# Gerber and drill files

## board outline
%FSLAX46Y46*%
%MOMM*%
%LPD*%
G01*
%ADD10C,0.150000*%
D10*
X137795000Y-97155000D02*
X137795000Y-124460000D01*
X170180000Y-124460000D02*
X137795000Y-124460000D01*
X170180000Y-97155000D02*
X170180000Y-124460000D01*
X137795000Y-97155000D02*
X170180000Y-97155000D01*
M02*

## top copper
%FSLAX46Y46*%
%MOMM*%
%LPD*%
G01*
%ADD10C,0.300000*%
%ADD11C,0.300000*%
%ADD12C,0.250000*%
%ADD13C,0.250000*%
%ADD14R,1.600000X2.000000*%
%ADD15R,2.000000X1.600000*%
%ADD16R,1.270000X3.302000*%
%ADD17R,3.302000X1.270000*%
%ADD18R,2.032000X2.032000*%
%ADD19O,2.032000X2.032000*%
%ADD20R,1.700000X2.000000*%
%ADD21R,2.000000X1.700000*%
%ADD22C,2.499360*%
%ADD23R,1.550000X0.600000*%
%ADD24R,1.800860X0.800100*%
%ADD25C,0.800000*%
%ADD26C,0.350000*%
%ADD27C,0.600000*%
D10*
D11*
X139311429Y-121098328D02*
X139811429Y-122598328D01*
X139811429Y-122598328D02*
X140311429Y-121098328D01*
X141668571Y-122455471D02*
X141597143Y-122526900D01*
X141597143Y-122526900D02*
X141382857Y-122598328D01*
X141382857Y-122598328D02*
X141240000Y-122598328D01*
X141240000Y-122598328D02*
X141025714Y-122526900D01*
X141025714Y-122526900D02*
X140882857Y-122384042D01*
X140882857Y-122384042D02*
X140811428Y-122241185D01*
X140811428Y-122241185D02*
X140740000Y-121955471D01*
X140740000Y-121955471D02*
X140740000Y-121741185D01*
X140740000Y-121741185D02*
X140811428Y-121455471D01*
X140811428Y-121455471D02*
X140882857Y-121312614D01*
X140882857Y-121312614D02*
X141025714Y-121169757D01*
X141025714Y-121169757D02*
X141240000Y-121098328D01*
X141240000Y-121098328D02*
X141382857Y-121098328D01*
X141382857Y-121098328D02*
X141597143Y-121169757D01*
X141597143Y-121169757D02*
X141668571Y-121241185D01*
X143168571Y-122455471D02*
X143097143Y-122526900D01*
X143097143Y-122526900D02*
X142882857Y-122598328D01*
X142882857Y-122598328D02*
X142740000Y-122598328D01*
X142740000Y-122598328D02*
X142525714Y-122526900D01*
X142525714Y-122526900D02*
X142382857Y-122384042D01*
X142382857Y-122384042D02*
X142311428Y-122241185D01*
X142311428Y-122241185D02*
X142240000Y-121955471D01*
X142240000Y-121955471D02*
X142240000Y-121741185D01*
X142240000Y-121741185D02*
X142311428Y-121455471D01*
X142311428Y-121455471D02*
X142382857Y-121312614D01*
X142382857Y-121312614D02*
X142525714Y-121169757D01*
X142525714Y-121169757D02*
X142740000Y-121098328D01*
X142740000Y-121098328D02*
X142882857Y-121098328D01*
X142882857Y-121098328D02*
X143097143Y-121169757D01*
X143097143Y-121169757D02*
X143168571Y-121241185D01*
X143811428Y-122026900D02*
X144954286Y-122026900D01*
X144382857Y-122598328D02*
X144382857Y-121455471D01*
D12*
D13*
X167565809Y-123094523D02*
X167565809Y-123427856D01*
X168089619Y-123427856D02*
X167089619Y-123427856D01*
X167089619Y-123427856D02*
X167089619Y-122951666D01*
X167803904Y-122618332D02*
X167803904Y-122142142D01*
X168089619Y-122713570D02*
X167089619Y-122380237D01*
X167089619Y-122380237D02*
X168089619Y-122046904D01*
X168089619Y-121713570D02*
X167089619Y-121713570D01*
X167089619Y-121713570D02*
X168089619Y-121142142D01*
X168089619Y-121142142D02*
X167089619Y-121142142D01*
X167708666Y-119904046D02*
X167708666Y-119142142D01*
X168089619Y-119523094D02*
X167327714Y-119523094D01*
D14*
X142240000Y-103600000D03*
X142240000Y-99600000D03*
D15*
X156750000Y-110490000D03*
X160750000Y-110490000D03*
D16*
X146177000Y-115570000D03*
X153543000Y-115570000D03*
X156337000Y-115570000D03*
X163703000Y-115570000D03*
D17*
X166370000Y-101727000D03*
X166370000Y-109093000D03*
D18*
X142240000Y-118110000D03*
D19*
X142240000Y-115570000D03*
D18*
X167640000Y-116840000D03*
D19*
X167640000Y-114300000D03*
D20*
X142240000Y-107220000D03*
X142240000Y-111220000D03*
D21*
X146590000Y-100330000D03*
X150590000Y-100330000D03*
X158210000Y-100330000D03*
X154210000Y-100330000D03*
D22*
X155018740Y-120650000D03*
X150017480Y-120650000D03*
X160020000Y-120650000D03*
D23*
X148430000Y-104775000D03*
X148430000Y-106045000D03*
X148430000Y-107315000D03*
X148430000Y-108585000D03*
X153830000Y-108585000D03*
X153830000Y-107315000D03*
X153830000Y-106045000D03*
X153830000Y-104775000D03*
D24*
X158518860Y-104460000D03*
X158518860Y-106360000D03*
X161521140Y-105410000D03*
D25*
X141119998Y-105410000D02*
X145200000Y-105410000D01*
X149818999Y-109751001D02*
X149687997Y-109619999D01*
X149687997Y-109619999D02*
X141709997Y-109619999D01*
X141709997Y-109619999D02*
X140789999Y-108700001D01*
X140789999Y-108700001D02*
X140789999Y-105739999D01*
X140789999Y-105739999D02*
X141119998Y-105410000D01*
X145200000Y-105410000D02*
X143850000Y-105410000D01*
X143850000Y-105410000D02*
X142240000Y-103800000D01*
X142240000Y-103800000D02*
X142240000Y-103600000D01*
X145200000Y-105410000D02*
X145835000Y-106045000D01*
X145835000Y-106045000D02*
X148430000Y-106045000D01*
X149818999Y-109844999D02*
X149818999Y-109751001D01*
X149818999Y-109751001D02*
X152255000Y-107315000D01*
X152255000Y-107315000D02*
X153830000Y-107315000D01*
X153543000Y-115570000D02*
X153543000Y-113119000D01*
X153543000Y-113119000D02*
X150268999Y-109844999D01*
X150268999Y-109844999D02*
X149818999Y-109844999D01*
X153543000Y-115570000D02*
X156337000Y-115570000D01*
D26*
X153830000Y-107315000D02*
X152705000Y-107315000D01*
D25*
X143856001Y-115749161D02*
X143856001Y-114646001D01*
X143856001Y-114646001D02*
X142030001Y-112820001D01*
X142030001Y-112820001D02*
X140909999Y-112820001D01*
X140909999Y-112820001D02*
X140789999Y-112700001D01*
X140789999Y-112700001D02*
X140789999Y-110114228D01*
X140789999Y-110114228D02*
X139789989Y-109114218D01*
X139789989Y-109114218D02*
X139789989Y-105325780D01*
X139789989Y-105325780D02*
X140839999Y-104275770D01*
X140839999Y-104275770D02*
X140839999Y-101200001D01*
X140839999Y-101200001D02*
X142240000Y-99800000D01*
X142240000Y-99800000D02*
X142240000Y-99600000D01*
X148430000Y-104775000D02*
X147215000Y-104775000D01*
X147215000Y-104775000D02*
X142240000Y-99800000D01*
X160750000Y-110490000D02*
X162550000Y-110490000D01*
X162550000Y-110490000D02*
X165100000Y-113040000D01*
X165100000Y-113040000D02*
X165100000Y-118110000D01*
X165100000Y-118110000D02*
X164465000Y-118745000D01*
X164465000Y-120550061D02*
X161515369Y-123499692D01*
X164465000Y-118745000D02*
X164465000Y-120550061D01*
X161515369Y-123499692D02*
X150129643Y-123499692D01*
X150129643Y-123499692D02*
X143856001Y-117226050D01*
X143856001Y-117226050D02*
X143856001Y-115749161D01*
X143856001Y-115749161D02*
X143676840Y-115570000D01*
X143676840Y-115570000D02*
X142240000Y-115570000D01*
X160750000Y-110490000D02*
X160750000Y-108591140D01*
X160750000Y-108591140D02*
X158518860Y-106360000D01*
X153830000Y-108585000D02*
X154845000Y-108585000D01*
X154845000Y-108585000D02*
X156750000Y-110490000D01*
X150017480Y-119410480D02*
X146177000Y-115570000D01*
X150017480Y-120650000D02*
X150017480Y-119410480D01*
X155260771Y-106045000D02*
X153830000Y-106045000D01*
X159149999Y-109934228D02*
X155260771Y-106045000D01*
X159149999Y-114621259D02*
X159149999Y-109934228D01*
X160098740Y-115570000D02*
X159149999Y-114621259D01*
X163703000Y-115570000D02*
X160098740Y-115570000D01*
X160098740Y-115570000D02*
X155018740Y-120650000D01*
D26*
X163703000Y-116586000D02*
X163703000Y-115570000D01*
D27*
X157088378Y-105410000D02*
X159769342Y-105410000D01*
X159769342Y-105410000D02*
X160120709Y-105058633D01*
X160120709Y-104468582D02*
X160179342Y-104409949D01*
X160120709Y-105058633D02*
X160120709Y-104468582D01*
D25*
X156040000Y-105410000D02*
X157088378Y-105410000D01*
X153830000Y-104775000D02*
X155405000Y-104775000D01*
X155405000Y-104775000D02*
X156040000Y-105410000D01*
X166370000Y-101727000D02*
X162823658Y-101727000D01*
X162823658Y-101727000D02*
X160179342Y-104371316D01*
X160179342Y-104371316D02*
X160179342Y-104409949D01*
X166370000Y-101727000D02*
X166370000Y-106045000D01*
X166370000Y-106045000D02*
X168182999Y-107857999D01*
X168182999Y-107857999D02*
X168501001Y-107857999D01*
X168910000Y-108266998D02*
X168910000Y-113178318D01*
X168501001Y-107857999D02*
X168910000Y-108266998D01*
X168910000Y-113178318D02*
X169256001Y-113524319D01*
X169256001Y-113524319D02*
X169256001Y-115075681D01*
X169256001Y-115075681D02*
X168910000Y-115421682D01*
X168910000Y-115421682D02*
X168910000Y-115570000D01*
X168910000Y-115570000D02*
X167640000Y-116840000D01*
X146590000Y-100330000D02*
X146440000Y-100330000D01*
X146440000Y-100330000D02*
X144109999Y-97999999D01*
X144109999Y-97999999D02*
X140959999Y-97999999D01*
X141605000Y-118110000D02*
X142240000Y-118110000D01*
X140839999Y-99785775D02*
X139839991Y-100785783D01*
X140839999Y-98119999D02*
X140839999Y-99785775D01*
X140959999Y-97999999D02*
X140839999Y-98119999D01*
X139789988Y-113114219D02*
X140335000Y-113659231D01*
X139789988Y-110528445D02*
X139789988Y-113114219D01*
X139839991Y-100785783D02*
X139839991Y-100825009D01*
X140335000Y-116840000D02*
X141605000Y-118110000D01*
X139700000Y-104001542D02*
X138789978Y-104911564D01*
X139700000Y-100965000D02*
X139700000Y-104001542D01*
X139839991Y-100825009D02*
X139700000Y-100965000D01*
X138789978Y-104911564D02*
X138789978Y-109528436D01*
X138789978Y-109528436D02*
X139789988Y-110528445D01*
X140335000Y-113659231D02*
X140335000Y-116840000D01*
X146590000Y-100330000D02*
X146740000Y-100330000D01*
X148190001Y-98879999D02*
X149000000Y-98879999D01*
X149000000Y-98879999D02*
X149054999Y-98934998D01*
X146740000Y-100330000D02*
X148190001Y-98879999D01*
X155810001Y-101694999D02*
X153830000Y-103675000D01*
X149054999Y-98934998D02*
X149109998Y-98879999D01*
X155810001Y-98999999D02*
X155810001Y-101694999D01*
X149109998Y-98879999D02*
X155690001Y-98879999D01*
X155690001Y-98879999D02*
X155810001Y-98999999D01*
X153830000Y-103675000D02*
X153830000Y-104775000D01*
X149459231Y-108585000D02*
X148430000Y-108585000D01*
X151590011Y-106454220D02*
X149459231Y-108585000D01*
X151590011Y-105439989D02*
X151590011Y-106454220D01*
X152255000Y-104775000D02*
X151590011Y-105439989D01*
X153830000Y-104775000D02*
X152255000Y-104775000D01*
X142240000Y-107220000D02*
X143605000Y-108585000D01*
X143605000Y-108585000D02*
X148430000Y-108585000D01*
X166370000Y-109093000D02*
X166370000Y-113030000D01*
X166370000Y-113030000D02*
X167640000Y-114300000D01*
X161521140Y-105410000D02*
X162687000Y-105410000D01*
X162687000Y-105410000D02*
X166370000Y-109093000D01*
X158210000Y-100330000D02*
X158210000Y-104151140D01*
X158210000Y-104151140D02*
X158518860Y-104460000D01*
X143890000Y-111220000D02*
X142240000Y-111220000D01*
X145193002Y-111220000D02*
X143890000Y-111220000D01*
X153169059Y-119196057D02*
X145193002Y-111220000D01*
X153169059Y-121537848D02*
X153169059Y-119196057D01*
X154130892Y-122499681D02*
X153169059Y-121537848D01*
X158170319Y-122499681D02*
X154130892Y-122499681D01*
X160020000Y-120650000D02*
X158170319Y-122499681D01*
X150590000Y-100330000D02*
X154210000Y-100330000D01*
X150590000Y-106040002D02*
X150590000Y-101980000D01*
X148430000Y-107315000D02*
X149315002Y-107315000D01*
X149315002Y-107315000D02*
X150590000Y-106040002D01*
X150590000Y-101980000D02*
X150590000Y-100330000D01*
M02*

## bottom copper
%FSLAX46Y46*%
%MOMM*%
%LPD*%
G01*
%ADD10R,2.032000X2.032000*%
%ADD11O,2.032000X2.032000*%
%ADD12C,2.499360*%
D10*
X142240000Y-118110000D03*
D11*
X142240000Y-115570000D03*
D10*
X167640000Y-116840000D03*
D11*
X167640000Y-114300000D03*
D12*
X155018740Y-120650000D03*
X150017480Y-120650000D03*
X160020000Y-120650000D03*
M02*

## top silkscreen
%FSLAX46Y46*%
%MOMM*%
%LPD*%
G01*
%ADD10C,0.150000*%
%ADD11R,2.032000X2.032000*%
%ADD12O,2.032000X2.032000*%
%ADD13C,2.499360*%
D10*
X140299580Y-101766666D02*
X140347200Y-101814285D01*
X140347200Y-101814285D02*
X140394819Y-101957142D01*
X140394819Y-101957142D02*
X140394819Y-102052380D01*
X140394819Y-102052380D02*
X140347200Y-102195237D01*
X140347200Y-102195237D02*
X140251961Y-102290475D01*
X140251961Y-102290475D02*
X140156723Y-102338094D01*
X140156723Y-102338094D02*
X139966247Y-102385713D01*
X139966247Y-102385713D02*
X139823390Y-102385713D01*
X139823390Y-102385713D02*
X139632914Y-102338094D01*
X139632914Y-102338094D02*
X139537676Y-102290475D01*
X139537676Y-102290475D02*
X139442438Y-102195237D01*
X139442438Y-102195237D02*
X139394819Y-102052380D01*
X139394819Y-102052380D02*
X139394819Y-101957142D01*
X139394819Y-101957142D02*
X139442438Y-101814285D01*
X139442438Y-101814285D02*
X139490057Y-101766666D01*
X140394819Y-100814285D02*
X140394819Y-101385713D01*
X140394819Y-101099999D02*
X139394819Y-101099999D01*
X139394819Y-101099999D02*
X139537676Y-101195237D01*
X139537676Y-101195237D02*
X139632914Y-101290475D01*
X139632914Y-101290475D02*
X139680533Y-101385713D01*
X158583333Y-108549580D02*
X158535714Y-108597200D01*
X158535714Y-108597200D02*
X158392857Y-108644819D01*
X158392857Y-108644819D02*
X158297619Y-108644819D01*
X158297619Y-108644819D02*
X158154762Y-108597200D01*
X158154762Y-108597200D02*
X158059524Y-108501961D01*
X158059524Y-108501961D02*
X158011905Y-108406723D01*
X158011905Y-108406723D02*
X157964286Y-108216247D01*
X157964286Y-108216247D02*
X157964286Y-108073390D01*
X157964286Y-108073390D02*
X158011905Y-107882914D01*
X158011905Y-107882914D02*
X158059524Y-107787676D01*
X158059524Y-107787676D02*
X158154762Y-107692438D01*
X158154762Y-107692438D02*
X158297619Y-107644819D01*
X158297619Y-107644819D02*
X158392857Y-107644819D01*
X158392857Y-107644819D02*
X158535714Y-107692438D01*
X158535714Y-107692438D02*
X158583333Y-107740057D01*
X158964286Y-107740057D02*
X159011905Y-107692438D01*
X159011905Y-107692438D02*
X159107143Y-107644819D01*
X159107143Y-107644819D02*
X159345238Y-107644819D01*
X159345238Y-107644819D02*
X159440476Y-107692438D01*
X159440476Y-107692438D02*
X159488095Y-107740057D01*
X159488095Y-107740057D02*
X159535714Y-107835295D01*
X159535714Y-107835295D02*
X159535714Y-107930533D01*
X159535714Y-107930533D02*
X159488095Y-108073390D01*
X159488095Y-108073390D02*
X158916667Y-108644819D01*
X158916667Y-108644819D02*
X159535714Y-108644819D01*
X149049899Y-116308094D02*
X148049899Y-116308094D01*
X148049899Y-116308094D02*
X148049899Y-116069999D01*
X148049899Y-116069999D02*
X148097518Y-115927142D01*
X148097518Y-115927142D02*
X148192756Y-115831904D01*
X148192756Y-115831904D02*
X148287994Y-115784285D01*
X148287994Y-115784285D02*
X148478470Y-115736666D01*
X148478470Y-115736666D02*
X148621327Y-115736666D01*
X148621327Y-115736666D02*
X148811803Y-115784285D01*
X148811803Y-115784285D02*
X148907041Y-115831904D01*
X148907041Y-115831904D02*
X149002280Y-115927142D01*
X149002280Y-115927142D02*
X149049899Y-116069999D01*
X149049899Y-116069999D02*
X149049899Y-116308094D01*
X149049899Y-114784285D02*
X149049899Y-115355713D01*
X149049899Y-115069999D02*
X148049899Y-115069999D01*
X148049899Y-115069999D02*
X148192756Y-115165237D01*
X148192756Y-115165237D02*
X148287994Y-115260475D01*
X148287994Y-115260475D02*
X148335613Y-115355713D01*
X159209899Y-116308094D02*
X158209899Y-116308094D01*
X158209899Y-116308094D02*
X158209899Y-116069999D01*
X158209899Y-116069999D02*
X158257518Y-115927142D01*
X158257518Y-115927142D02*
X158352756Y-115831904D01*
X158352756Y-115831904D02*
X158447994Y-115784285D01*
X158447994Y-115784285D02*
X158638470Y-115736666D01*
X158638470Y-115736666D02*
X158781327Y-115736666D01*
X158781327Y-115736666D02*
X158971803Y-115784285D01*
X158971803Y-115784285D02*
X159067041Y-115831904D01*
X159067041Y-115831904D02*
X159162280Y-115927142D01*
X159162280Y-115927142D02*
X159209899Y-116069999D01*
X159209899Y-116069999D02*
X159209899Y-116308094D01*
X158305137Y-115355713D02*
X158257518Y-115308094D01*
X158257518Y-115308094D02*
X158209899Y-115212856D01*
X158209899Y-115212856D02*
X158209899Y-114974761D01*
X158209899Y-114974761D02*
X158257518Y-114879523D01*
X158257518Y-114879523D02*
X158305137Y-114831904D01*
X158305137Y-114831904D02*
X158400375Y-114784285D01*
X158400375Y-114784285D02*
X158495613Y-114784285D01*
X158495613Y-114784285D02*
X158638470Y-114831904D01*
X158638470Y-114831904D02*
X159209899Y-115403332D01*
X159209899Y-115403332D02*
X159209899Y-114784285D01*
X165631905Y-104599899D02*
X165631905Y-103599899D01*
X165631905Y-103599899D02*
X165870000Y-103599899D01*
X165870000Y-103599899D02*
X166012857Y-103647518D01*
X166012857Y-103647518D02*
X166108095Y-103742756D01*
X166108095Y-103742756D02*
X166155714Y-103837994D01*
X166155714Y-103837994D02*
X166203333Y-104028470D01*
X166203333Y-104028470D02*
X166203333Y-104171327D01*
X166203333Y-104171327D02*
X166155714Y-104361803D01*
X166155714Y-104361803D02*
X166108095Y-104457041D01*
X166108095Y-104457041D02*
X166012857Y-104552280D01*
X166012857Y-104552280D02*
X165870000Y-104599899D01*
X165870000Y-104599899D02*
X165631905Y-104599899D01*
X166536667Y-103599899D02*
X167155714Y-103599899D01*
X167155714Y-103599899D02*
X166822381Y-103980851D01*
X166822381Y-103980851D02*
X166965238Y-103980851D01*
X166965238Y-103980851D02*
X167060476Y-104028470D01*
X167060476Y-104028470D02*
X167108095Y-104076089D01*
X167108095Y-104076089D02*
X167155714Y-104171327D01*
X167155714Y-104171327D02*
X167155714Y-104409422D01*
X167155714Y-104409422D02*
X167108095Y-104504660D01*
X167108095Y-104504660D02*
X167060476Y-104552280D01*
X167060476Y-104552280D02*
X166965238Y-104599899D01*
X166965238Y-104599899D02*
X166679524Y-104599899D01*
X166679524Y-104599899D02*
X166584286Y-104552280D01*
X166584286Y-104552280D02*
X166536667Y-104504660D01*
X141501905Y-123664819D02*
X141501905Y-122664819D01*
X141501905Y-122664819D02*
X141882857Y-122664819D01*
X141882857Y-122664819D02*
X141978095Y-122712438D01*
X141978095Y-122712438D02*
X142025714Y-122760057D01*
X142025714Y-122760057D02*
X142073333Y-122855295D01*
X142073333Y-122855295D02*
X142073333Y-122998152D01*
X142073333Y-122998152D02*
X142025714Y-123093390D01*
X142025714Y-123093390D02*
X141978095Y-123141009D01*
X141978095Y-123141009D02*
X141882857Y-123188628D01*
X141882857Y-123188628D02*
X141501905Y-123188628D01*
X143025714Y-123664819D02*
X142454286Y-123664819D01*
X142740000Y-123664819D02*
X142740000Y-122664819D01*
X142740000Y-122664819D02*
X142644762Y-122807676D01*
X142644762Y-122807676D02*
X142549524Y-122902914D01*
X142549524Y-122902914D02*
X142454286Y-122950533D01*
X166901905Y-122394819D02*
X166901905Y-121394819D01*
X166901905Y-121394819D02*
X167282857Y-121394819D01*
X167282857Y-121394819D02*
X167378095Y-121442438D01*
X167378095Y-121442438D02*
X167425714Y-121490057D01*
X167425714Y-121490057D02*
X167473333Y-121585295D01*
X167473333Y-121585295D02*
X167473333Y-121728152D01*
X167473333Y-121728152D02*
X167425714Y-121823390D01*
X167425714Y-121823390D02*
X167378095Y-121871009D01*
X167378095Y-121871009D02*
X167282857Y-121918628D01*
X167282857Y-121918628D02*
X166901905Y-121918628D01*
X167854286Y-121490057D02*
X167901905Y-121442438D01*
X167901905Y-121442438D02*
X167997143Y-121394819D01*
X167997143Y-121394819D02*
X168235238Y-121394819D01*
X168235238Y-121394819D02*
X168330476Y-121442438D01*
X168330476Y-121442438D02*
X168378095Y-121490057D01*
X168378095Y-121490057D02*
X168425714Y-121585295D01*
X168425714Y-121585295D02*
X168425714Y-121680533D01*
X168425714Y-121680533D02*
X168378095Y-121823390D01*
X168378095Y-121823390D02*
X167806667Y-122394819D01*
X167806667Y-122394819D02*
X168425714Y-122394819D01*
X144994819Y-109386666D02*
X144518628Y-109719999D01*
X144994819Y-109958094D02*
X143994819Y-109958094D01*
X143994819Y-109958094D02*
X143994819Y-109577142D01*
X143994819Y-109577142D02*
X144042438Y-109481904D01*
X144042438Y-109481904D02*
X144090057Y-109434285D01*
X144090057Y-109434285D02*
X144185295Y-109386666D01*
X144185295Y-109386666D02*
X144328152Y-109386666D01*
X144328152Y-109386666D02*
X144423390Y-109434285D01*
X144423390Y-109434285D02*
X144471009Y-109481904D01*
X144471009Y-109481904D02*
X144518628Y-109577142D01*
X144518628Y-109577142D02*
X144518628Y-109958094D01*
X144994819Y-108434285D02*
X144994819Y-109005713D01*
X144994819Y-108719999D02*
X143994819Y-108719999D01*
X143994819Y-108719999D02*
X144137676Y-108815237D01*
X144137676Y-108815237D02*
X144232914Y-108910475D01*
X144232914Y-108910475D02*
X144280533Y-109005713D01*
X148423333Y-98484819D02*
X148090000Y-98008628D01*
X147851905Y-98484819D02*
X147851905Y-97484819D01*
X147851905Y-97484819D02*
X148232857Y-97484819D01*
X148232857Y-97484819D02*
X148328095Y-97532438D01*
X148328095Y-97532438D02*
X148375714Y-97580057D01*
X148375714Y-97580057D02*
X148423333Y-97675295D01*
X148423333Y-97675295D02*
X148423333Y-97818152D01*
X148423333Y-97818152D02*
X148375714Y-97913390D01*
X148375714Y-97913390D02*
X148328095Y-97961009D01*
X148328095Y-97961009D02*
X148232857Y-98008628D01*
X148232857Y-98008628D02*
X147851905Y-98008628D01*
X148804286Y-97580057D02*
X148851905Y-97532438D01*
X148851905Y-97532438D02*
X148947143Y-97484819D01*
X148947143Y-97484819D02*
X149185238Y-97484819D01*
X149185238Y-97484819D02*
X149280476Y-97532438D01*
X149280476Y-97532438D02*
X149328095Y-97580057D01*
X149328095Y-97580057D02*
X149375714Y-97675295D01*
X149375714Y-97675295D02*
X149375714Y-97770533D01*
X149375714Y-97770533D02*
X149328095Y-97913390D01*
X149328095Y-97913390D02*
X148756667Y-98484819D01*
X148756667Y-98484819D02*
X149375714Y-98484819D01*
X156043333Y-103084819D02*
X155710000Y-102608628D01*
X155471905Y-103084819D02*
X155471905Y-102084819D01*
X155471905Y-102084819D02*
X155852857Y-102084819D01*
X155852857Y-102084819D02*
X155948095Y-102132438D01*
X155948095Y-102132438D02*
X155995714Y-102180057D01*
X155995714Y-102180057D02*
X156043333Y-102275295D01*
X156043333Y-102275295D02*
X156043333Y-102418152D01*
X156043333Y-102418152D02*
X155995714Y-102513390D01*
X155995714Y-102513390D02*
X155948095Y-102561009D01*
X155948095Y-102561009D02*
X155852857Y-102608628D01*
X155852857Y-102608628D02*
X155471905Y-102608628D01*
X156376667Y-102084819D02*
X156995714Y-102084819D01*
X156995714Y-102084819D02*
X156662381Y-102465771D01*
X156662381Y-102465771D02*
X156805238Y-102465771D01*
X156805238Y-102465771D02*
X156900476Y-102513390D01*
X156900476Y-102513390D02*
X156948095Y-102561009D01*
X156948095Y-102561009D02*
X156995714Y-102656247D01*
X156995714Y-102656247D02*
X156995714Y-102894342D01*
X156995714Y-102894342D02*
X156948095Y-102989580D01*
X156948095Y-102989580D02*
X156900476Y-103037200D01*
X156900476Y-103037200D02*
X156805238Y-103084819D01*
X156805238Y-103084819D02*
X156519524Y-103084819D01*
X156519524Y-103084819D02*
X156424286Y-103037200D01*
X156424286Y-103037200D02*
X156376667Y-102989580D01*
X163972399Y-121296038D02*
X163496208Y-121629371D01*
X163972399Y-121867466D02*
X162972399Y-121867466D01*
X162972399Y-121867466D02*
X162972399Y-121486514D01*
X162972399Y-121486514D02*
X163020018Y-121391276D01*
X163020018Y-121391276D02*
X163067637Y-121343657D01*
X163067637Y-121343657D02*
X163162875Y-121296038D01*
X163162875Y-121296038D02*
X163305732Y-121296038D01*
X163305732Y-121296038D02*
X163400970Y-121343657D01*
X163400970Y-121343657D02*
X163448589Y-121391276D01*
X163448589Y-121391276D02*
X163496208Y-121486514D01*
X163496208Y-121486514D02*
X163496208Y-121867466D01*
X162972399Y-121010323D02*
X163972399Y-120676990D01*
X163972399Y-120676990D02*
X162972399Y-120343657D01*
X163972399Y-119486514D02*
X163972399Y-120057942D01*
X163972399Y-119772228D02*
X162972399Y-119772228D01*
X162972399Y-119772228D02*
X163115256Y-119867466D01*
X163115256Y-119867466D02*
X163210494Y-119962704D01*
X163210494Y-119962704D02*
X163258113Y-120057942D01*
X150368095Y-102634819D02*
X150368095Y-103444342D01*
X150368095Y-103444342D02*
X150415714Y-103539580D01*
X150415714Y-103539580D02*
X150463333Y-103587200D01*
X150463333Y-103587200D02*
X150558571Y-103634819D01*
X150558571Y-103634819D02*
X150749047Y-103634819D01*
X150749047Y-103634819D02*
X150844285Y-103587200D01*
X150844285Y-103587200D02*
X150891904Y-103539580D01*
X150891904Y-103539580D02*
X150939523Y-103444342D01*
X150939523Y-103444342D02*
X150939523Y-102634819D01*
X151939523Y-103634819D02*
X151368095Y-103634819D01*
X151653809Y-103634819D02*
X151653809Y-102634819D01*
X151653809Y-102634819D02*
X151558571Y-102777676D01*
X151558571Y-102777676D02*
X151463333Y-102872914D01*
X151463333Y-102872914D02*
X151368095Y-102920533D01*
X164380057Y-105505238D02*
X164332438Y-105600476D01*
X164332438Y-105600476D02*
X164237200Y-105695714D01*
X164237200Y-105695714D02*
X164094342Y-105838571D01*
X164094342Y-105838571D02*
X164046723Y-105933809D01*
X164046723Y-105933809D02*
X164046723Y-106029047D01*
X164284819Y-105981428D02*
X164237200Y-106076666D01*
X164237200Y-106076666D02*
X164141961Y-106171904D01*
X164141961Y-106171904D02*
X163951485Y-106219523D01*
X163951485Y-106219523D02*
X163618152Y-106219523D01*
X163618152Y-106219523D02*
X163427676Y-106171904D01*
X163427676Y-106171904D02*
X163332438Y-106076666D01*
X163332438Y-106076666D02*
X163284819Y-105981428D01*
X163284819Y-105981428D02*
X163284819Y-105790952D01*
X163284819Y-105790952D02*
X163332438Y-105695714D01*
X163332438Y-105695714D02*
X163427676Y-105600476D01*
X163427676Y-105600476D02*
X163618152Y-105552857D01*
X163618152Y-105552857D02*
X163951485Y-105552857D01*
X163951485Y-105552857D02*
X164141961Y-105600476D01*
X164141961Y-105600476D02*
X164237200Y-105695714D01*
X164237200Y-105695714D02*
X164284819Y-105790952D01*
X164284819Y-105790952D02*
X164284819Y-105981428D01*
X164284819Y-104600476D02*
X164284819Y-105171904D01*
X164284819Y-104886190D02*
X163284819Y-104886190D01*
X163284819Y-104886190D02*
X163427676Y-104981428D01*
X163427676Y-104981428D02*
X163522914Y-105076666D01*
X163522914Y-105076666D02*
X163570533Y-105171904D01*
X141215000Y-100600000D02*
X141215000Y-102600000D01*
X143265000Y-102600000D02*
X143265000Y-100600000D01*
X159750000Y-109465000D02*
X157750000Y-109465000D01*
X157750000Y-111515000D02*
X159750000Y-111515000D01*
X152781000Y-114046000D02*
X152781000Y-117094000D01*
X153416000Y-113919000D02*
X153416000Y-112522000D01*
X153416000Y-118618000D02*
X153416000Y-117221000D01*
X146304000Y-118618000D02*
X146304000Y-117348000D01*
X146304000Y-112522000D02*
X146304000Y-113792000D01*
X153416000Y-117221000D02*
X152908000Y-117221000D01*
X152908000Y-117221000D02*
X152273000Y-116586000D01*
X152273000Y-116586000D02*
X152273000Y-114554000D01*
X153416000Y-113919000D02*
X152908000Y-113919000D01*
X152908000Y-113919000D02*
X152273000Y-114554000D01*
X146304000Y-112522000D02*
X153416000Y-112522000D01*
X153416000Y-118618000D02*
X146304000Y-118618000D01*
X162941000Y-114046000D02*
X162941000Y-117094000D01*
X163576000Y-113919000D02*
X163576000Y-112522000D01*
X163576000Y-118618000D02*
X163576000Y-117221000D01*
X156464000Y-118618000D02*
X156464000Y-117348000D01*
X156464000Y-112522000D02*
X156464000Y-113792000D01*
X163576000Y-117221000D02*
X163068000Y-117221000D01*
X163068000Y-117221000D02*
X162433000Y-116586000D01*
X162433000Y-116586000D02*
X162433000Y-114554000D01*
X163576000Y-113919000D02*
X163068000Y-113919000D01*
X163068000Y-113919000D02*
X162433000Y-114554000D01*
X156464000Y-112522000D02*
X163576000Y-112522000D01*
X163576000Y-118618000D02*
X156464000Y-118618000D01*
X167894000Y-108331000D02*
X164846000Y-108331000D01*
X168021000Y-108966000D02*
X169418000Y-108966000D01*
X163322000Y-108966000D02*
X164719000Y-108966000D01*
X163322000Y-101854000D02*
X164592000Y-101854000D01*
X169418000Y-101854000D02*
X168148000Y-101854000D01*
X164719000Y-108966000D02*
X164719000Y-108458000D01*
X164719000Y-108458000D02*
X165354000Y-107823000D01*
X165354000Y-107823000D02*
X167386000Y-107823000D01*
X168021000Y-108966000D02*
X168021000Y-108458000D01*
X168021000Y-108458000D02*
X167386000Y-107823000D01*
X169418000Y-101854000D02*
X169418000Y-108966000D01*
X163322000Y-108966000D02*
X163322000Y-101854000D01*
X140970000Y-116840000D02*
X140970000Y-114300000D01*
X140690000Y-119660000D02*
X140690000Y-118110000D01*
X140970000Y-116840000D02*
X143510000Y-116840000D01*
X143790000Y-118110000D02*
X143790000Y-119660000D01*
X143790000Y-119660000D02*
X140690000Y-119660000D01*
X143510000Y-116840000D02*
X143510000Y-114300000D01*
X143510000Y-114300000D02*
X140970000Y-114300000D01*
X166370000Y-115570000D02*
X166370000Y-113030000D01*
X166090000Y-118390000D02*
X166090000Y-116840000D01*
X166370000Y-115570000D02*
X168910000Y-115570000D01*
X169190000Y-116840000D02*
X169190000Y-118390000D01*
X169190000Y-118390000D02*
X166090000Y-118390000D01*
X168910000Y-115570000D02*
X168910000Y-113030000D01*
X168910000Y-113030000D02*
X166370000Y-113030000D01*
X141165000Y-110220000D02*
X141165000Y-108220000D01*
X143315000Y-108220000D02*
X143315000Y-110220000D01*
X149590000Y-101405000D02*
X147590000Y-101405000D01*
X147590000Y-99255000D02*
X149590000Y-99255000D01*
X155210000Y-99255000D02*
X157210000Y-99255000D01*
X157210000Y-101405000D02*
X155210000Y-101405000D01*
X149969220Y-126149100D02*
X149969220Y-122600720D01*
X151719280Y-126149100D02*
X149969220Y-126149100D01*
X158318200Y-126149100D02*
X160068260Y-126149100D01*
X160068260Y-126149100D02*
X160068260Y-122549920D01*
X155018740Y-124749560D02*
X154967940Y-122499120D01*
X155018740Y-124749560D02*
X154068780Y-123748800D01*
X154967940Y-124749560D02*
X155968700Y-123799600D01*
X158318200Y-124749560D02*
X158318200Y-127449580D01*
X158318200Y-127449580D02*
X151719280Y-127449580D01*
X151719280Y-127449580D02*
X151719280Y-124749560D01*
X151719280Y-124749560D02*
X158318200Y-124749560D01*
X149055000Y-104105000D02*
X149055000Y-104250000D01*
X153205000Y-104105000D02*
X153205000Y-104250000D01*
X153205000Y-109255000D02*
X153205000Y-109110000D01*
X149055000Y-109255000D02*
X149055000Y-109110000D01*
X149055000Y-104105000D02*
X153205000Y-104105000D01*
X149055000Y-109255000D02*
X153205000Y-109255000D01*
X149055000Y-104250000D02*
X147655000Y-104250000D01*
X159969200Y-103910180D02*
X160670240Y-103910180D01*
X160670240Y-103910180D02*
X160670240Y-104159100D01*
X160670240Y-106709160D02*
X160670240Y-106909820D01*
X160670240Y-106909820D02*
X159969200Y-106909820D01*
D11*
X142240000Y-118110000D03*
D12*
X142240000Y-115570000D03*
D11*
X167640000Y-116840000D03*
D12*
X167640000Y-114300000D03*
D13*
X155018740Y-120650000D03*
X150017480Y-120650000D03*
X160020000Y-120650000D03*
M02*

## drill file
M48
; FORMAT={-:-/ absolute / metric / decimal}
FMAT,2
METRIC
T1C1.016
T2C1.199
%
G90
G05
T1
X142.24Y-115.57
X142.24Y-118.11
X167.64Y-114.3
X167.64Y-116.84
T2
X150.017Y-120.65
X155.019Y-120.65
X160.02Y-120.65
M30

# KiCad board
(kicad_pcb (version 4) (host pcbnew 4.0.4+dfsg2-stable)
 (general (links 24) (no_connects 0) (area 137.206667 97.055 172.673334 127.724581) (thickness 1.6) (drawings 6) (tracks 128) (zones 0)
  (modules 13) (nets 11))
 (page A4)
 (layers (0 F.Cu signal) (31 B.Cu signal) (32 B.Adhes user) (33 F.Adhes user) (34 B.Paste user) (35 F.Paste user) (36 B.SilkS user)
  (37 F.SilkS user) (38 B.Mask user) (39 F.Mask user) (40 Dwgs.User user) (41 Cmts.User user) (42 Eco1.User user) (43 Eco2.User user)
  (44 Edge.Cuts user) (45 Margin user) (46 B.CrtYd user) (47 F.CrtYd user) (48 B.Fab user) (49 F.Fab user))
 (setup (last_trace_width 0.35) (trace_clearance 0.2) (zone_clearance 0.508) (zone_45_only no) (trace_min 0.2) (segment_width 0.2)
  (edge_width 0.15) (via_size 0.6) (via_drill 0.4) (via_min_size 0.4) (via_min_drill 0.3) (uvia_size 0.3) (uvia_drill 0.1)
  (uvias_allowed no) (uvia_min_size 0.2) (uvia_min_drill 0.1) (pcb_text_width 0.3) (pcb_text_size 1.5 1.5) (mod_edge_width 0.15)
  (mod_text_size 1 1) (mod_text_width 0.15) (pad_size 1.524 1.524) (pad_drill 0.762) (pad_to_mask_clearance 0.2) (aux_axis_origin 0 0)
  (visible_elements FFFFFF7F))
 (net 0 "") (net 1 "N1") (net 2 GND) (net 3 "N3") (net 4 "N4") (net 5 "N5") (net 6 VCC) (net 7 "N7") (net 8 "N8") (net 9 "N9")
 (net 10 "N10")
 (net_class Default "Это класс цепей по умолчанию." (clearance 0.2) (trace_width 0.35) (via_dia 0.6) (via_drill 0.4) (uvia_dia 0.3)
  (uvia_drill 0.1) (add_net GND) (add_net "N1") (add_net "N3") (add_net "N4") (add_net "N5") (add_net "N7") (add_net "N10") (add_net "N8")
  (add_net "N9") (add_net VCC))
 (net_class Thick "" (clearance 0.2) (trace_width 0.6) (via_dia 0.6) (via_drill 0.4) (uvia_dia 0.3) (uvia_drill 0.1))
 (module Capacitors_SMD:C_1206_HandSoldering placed (layer F.Cu) (at 142.24 101.6 90)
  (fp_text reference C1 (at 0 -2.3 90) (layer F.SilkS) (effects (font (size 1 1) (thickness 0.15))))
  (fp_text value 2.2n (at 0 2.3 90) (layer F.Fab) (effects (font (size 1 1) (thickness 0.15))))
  (fp_line (start 1 -1.025) (end -1 -1.025) (layer F.SilkS) (width 0.15))
  (fp_line (start -1 1.025) (end 1 1.025) (layer F.SilkS) (width 0.15))
  (pad 1 smd rect (at -2 0 90) (size 2 1.6) (layers F.Cu F.Paste F.Mask) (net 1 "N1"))
  (pad 2 smd rect (at 2 0 90) (size 2 1.6) (layers F.Cu F.Paste F.Mask) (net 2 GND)))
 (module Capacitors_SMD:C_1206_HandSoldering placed (layer F.Cu) (at 158.75 110.49)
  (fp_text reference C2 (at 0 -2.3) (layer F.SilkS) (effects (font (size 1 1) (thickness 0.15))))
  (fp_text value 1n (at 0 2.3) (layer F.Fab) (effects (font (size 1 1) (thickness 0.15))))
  (fp_line (start 1 -1.025) (end -1 -1.025) (layer F.SilkS) (width 0.15))
  (fp_line (start -1 1.025) (end 1 1.025) (layer F.SilkS) (width 0.15))
  (pad 1 smd rect (at -2 0) (size 2 1.6) (layers F.Cu F.Paste F.Mask) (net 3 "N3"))
  (pad 2 smd rect (at 2 0) (size 2 1.6) (layers F.Cu F.Paste F.Mask) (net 2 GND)))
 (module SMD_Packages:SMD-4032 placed (layer F.Cu) (at 149.86 115.57)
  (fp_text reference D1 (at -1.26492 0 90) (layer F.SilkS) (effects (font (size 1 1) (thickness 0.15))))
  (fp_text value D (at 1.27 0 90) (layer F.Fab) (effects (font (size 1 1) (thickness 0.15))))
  (fp_line (start 2.921 -1.524) (end 2.921 1.524) (layer F.SilkS) (width 0.15))
  (fp_line (start 3.556 -1.651) (end 3.556 -3.048) (layer F.SilkS) (width 0.15))
  (fp_line (start 3.556 3.048) (end 3.556 1.651) (layer F.SilkS) (width 0.15))
  (fp_line (start -3.556 3.048) (end -3.556 1.778) (layer F.SilkS) (width 0.15))
  (fp_line (start -3.556 -3.048) (end -3.556 -1.778) (layer F.SilkS) (width 0.15))
  (fp_line (start 3.556 1.651) (end 3.048 1.651) (layer F.SilkS) (width 0.15))
  (fp_line (start 3.048 1.651) (end 2.413 1.016) (layer F.SilkS) (width 0.15))
  (fp_line (start 2.413 1.016) (end 2.413 -1.016) (layer F.SilkS) (width 0.15))
  (fp_line (start 3.556 -1.651) (end 3.048 -1.651) (layer F.SilkS) (width 0.15))
  (fp_line (start 3.048 -1.651) (end 2.413 -1.016) (layer F.SilkS) (width 0.15))
  (fp_line (start -3.556 -3.048) (end 3.556 -3.048) (layer F.SilkS) (width 0.15))
  (fp_line (start 3.556 3.048) (end -3.556 3.048) (layer F.SilkS) (width 0.15))
  (pad 1 smd rect (at -3.683 0) (size 1.27 3.302) (layers F.Cu F.Paste F.Mask) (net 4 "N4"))
  (pad 2 smd rect (at 3.683 0) (size 1.27 3.302) (layers F.Cu F.Paste F.Mask) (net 1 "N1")))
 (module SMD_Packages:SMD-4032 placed (layer F.Cu) (at 160.02 115.57)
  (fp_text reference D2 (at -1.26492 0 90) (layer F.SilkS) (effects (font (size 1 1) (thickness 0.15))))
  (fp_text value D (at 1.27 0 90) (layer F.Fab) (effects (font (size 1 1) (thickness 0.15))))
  (fp_line (start 2.921 -1.524) (end 2.921 1.524) (layer F.SilkS) (width 0.15))
  (fp_line (start 3.556 -1.651) (end 3.556 -3.048) (layer F.SilkS) (width 0.15))
  (fp_line (start 3.556 3.048) (end 3.556 1.651) (layer F.SilkS) (width 0.15))
  (fp_line (start -3.556 3.048) (end -3.556 1.778) (layer F.SilkS) (width 0.15))
  (fp_line (start -3.556 -3.048) (end -3.556 -1.778) (layer F.SilkS) (width 0.15))
  (fp_line (start 3.556 1.651) (end 3.048 1.651) (layer F.SilkS) (width 0.15))
  (fp_line (start 3.048 1.651) (end 2.413 1.016) (layer F.SilkS) (width 0.15))
  (fp_line (start 2.413 1.016) (end 2.413 -1.016) (layer F.SilkS) (width 0.15))
  (fp_line (start 3.556 -1.651) (end 3.048 -1.651) (layer F.SilkS) (width 0.15))
  (fp_line (start 3.048 -1.651) (end 2.413 -1.016) (layer F.SilkS) (width 0.15))
  (fp_line (start -3.556 -3.048) (end 3.556 -3.048) (layer F.SilkS) (width 0.15))
  (fp_line (start 3.556 3.048) (end -3.556 3.048) (layer F.SilkS) (width 0.15))
  (pad 1 smd rect (at -3.683 0) (size 1.27 3.302) (layers F.Cu F.Paste F.Mask) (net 1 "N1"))
  (pad 2 smd rect (at 3.683 0) (size 1.27 3.302) (layers F.Cu F.Paste F.Mask) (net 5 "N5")))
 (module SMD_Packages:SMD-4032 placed (layer F.Cu) (at 166.37 105.41 270)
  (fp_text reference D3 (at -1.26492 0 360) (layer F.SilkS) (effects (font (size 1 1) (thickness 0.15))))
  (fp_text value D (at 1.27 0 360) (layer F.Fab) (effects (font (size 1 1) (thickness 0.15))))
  (fp_line (start 2.921 -1.524) (end 2.921 1.524) (layer F.SilkS) (width 0.15))
  (fp_line (start 3.556 -1.651) (end 3.556 -3.048) (layer F.SilkS) (width 0.15))
  (fp_line (start 3.556 3.048) (end 3.556 1.651) (layer F.SilkS) (width 0.15))
  (fp_line (start -3.556 3.048) (end -3.556 1.778) (layer F.SilkS) (width 0.15))
  (fp_line (start -3.556 -3.048) (end -3.556 -1.778) (layer F.SilkS) (width 0.15))
  (fp_line (start 3.556 1.651) (end 3.048 1.651) (layer F.SilkS) (width 0.15))
  (fp_line (start 3.048 1.651) (end 2.413 1.016) (layer F.SilkS) (width 0.15))
  (fp_line (start 2.413 1.016) (end 2.413 -1.016) (layer F.SilkS) (width 0.15))
  (fp_line (start 3.556 -1.651) (end 3.048 -1.651) (layer F.SilkS) (width 0.15))
  (fp_line (start 3.048 -1.651) (end 2.413 -1.016) (layer F.SilkS) (width 0.15))
  (fp_line (start -3.556 -3.048) (end 3.556 -3.048) (layer F.SilkS) (width 0.15))
  (fp_line (start 3.556 3.048) (end -3.556 3.048) (layer F.SilkS) (width 0.15))
  (pad 1 smd rect (at -3.683 0 270) (size 1.27 3.302) (layers F.Cu F.Paste F.Mask) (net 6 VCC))
  (pad 2 smd rect (at 3.683 0 270) (size 1.27 3.302) (layers F.Cu F.Paste F.Mask) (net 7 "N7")))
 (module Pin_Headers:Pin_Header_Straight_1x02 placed (layer F.Cu) (at 142.24 118.11 180)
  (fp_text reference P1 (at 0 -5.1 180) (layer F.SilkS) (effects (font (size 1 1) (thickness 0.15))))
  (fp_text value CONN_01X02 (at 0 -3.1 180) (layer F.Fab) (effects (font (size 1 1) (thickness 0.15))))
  (fp_line (start 1.27 1.27) (end 1.27 3.81) (layer F.SilkS) (width 0.15))
  (fp_line (start 1.55 -1.55) (end 1.55 0) (layer F.SilkS) (width 0.15))
  (fp_line (start 1.27 1.27) (end -1.27 1.27) (layer F.SilkS) (width 0.15))
  (fp_line (start -1.55 0) (end -1.55 -1.55) (layer F.SilkS) (width 0.15))
  (fp_line (start -1.55 -1.55) (end 1.55 -1.55) (layer F.SilkS) (width 0.15))
  (fp_line (start -1.27 1.27) (end -1.27 3.81) (layer F.SilkS) (width 0.15))
  (fp_line (start -1.27 3.81) (end 1.27 3.81) (layer F.SilkS) (width 0.15))
  (pad 1 thru_hole rect (at 0 0 180) (size 2.032 2.032) (drill 1.016) (layers *.Cu *.Mask F.SilkS) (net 6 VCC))
  (pad 2 thru_hole oval (at 0 2.54 180) (size 2.032 2.032) (drill 1.016) (layers *.Cu *.Mask F.SilkS) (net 2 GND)))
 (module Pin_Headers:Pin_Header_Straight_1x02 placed (layer F.Cu) (at 167.64 116.84 180)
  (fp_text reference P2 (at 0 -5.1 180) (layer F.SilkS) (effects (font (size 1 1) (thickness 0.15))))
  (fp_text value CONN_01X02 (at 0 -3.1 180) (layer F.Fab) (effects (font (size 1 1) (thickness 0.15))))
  (fp_line (start 1.27 1.27) (end 1.27 3.81) (layer F.SilkS) (width 0.15))
  (fp_line (start 1.55 -1.55) (end 1.55 0) (layer F.SilkS) (width 0.15))
  (fp_line (start 1.27 1.27) (end -1.27 1.27) (layer F.SilkS) (width 0.15))
  (fp_line (start -1.55 0) (end -1.55 -1.55) (layer F.SilkS) (width 0.15))
  (fp_line (start -1.55 -1.55) (end 1.55 -1.55) (layer F.SilkS) (width 0.15))
  (fp_line (start -1.27 1.27) (end -1.27 3.81) (layer F.SilkS) (width 0.15))
  (fp_line (start -1.27 3.81) (end 1.27 3.81) (layer F.SilkS) (width 0.15))
  (pad 1 thru_hole rect (at 0 0 180) (size 2.032 2.032) (drill 1.016) (layers *.Cu *.Mask F.SilkS) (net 6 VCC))
  (pad 2 thru_hole oval (at 0 2.54 180) (size 2.032 2.032) (drill 1.016) (layers *.Cu *.Mask F.SilkS) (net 7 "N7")))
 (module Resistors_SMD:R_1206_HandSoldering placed (layer F.Cu) (at 142.24 109.22 270)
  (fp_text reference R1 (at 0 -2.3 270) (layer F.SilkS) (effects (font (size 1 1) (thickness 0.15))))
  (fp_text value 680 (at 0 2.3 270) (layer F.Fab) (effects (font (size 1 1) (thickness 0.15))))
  (fp_line (start 1 1.075) (end -1 1.075) (layer F.SilkS) (width 0.15))
  (fp_line (start -1 -1.075) (end 1 -1.075) (layer F.SilkS) (width 0.15))
  (pad 1 smd rect (at -2 0 270) (size 2 1.7) (layers F.Cu F.Paste F.Mask) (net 6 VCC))
  (pad 2 smd rect (at 2 0 270) (size 2 1.7) (layers F.Cu F.Paste F.Mask) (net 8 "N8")))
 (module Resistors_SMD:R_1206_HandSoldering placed (layer F.Cu) (at 148.59 100.33)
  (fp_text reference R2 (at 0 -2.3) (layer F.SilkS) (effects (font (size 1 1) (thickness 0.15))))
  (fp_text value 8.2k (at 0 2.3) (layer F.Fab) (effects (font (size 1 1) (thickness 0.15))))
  (fp_line (start 1 1.075) (end -1 1.075) (layer F.SilkS) (width 0.15))
  (fp_line (start -1 -1.075) (end 1 -1.075) (layer F.SilkS) (width 0.15))
  (pad 1 smd rect (at -2 0) (size 2 1.7) (layers F.Cu F.Paste F.Mask) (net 6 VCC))
  (pad 2 smd rect (at 2 0) (size 2 1.7) (layers F.Cu F.Paste F.Mask) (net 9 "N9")))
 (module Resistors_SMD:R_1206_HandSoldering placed (layer F.Cu) (at 156.21 100.33 180)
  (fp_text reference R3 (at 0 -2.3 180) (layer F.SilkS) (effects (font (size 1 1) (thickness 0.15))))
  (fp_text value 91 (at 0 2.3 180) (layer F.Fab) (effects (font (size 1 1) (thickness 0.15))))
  (fp_line (start 1 1.075) (end -1 1.075) (layer F.SilkS) (width 0.15))
  (fp_line (start -1 -1.075) (end 1 -1.075) (layer F.SilkS) (width 0.15))
  (pad 1 smd rect (at -2 0 180) (size 2 1.7) (layers F.Cu F.Paste F.Mask) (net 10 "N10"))
  (pad 2 smd rect (at 2 0 180) (size 2 1.7) (layers F.Cu F.Paste F.Mask) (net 9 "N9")))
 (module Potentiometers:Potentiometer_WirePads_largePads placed (layer F.Cu) (at 160.02 120.65 270)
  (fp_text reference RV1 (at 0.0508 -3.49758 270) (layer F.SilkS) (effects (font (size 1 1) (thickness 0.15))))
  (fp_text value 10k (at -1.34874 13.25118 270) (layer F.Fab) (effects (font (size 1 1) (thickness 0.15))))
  (fp_line (start 5.4991 10.05078) (end 1.95072 10.05078) (layer F.SilkS) (width 0.15))
  (fp_line (start 5.4991 8.30072) (end 5.4991 10.05078) (layer F.SilkS) (width 0.15))
  (fp_line (start 5.4991 1.7018) (end 5.4991 -0.04826) (layer F.SilkS) (width 0.15))
  (fp_line (start 5.4991 -0.04826) (end 1.89992 -0.04826) (layer F.SilkS) (width 0.15))
  (fp_line (start 4.09956 5.00126) (end 1.84912 5.05206) (layer F.SilkS) (width 0.15))
  (fp_line (start 4.09956 5.00126) (end 3.0988 5.95122) (layer F.SilkS) (width 0.15))
  (fp_line (start 4.09956 5.05206) (end 3.1496 4.0513) (layer F.SilkS) (width 0.15))
  (fp_line (start 4.09956 1.7018) (end 6.79958 1.7018) (layer F.SilkS) (width 0.15))
  (fp_line (start 6.79958 1.7018) (end 6.79958 8.30072) (layer F.SilkS) (width 0.15))
  (fp_line (start 6.79958 8.30072) (end 4.09956 8.30072) (layer F.SilkS) (width 0.15))
  (fp_line (start 4.09956 8.30072) (end 4.09956 1.7018) (layer F.SilkS) (width 0.15))
  (pad 2 thru_hole circle (at 0 5.00126 270) (size 2.49936 2.49936) (drill 1.19888) (layers *.Cu *.Mask F.SilkS) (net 5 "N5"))
  (pad 3 thru_hole circle (at 0 10.00252 270) (size 2.49936 2.49936) (drill 1.19888) (layers *.Cu *.Mask F.SilkS) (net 4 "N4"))
  (pad 1 thru_hole circle (at 0 0 270) (size 2.49936 2.49936) (drill 1.19888) (layers *.Cu *.Mask F.SilkS) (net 8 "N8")))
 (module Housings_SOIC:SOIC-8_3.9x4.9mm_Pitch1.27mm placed (layer F.Cu) (at 151.13 106.68)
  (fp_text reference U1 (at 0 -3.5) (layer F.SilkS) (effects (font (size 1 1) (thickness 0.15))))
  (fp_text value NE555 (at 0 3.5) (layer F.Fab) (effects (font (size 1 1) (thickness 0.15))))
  (fp_line (start -2.075 -2.575) (end -2.075 -2.43) (layer F.SilkS) (width 0.15))
  (fp_line (start 2.075 -2.575) (end 2.075 -2.43) (layer F.SilkS) (width 0.15))
  (fp_line (start 2.075 2.575) (end 2.075 2.43) (layer F.SilkS) (width 0.15))
  (fp_line (start -2.075 2.575) (end -2.075 2.43) (layer F.SilkS) (width 0.15))
  (fp_line (start -2.075 -2.575) (end 2.075 -2.575) (layer F.SilkS) (width 0.15))
  (fp_line (start -2.075 2.575) (end 2.075 2.575) (layer F.SilkS) (width 0.15))
  (fp_line (start -2.075 -2.43) (end -3.475 -2.43) (layer F.SilkS) (width 0.15))
  (pad 1 smd rect (at -2.7 -1.905) (size 1.55 0.6) (layers F.Cu F.Paste F.Mask) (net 2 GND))
  (pad 2 smd rect (at -2.7 -0.635) (size 1.55 0.6) (layers F.Cu F.Paste F.Mask) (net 1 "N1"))
  (pad 3 smd rect (at -2.7 0.635) (size 1.55 0.6) (layers F.Cu F.Paste F.Mask) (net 9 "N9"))
  (pad 4 smd rect (at -2.7 1.905) (size 1.55 0.6) (layers F.Cu F.Paste F.Mask) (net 6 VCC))
  (pad 5 smd rect (at 2.7 1.905) (size 1.55 0.6) (layers F.Cu F.Paste F.Mask) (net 3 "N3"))
  (pad 6 smd rect (at 2.7 0.635) (size 1.55 0.6) (layers F.Cu F.Paste F.Mask) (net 1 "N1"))
  (pad 7 smd rect (at 2.7 -0.635) (size 1.55 0.6) (layers F.Cu F.Paste F.Mask) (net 5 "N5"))
  (pad 8 smd rect (at 2.7 -1.905) (size 1.55 0.6) (layers F.Cu F.Paste F.Mask) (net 6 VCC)))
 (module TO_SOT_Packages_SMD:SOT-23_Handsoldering (layer F.Cu) (at 160.02 105.41 270)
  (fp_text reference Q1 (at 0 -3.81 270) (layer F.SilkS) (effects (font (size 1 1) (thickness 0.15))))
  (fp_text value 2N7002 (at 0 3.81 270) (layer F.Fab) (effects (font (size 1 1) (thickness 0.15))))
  (fp_line (start -1.49982 0.0508) (end -1.49982 -0.65024) (layer F.SilkS) (width 0.15))
  (fp_line (start -1.49982 -0.65024) (end -1.2509 -0.65024) (layer F.SilkS) (width 0.15))
  (fp_line (start 1.29916 -0.65024) (end 1.49982 -0.65024) (layer F.SilkS) (width 0.15))
  (fp_line (start 1.49982 -0.65024) (end 1.49982 0.0508) (layer F.SilkS) (width 0.15))
  (pad 1 smd rect (at -0.95 1.50114 270) (size 0.8001 1.80086) (layers F.Cu F.Paste F.Mask) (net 10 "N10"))
  (pad 2 smd rect (at 0.95 1.50114 270) (size 0.8001 1.80086) (layers F.Cu F.Paste F.Mask) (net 2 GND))
  (pad 3 smd rect (at 0 -1.50114 270) (size 0.8001 1.80086) (layers F.Cu F.Paste F.Mask) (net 7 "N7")))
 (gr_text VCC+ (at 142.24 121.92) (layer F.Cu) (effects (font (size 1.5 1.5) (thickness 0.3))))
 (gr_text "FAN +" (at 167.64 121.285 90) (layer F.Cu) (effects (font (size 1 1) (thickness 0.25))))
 (gr_line (start 137.795 97.155) (end 137.795 124.46) (layer Edge.Cuts) (width 0.15))
 (gr_line (start 170.18 124.46) (end 137.795 124.46) (layer Edge.Cuts) (width 0.15))
 (gr_line (start 170.18 97.155) (end 170.18 124.46) (layer Edge.Cuts) (width 0.15))
 (gr_line (start 137.795 97.155) (end 170.18 97.155) (layer Edge.Cuts) (width 0.15))
 (segment (start 141.119998 105.41) (end 145.2 105.41) (width 0.8) (layer F.Cu) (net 1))
 (segment (start 149.818999 109.751001) (end 149.687997 109.619999) (width 0.8) (layer F.Cu) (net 1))
 (segment (start 149.687997 109.619999) (end 141.709997 109.619999) (width 0.8) (layer F.Cu) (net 1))
 (segment (start 141.709997 109.619999) (end 140.789999 108.700001) (width 0.8) (layer F.Cu) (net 1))
 (segment (start 140.789999 108.700001) (end 140.789999 105.739999) (width 0.8) (layer F.Cu) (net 1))
 (segment (start 140.789999 105.739999) (end 141.119998 105.41) (width 0.8) (layer F.Cu) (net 1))
 (segment (start 145.2 105.41) (end 143.85 105.41) (width 0.8) (layer F.Cu) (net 1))
 (segment (start 143.85 105.41) (end 142.24 103.8) (width 0.8) (layer F.Cu) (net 1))
 (segment (start 142.24 103.8) (end 142.24 103.6) (width 0.8) (layer F.Cu) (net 1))
 (segment (start 145.2 105.41) (end 145.835 106.045) (width 0.8) (layer F.Cu) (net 1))
 (segment (start 145.835 106.045) (end 148.43 106.045) (width 0.8) (layer F.Cu) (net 1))
 (segment (start 149.818999 109.844999) (end 149.818999 109.751001) (width 0.8) (layer F.Cu) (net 1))
 (segment (start 149.818999 109.751001) (end 152.255 107.315) (width 0.8) (layer F.Cu) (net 1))
 (segment (start 152.255 107.315) (end 153.83 107.315) (width 0.8) (layer F.Cu) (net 1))
 (segment (start 153.543 115.57) (end 153.543 113.119) (width 0.8) (layer F.Cu) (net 1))
 (segment (start 153.543 113.119) (end 150.268999 109.844999) (width 0.8) (layer F.Cu) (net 1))
 (segment (start 150.268999 109.844999) (end 149.818999 109.844999) (width 0.8) (layer F.Cu) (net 1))
 (segment (start 153.543 115.57) (end 156.337 115.57) (width 0.8) (layer F.Cu) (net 1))
 (segment (start 153.83 107.315) (end 152.705 107.315) (width 0.35) (layer F.Cu) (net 1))
 (segment (start 143.856001 115.749161) (end 143.856001 114.646001) (width 0.8) (layer F.Cu) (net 2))
 (segment (start 143.856001 114.646001) (end 142.030001 112.820001) (width 0.8) (layer F.Cu) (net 2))
 (segment (start 142.030001 112.820001) (end 140.909999 112.820001) (width 0.8) (layer F.Cu) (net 2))
 (segment (start 140.909999 112.820001) (end 140.789999 112.700001) (width 0.8) (layer F.Cu) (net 2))
 (segment (start 140.789999 112.700001) (end 140.789999 110.114228) (width 0.8) (layer F.Cu) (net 2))
 (segment (start 140.789999 110.114228) (end 139.789989 109.114218) (width 0.8) (layer F.Cu) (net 2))
 (segment (start 139.789989 109.114218) (end 139.789989 105.32578) (width 0.8) (layer F.Cu) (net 2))
 (segment (start 139.789989 105.32578) (end 140.839999 104.27577) (width 0.8) (layer F.Cu) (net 2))
 (segment (start 140.839999 104.27577) (end 140.839999 101.200001) (width 0.8) (layer F.Cu) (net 2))
 (segment (start 140.839999 101.200001) (end 142.24 99.8) (width 0.8) (layer F.Cu) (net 2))
 (segment (start 142.24 99.8) (end 142.24 99.6) (width 0.8) (layer F.Cu) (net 2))
 (segment (start 148.43 104.775) (end 147.215 104.775) (width 0.8) (layer F.Cu) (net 2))
 (segment (start 147.215 104.775) (end 142.24 99.8) (width 0.8) (layer F.Cu) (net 2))
 (segment (start 160.75 110.49) (end 162.55 110.49) (width 0.8) (layer F.Cu) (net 2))
 (segment (start 162.55 110.49) (end 165.1 113.04) (width 0.8) (layer F.Cu) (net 2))
 (segment (start 165.1 113.04) (end 165.1 118.11) (width 0.8) (layer F.Cu) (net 2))
 (segment (start 165.1 118.11) (end 164.465 118.745) (width 0.8) (layer F.Cu) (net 2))
 (segment (start 164.465 120.550061) (end 161.515369 123.499692) (width 0.8) (layer F.Cu) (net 2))
 (segment (start 164.465 118.745) (end 164.465 120.550061) (width 0.8) (layer F.Cu) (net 2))
 (segment (start 161.515369 123.499692) (end 150.129643 123.499692) (width 0.8) (layer F.Cu) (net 2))
 (segment (start 150.129643 123.499692) (end 143.856001 117.22605) (width 0.8) (layer F.Cu) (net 2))
 (segment (start 143.856001 117.22605) (end 143.856001 115.749161) (width 0.8) (layer F.Cu) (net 2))
 (segment (start 143.856001 115.749161) (end 143.67684 115.57) (width 0.8) (layer F.Cu) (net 2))
 (segment (start 143.67684 115.57) (end 142.24 115.57) (width 0.8) (layer F.Cu) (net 2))
 (segment (start 160.75 110.49) (end 160.75 108.59114) (width 0.8) (layer F.Cu) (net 2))
 (segment (start 160.75 108.59114) (end 158.51886 106.36) (width 0.8) (layer F.Cu) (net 2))
 (segment (start 153.83 108.585) (end 154.845 108.585) (width 0.8) (layer F.Cu) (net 3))
 (segment (start 154.845 108.585) (end 156.75 110.49) (width 0.8) (layer F.Cu) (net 3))
 (segment (start 150.01748 119.41048) (end 146.177 115.57) (width 0.8) (layer F.Cu) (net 4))
 (segment (start 150.01748 120.65) (end 150.01748 119.41048) (width 0.8) (layer F.Cu) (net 4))
 (segment (start 155.260771 106.045) (end 153.83 106.045) (width 0.8) (layer F.Cu) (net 5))
 (segment (start 159.149999 109.934228) (end 155.260771 106.045) (width 0.8) (layer F.Cu) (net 5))
 (segment (start 159.149999 114.621259) (end 159.149999 109.934228) (width 0.8) (layer F.Cu) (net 5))
 (segment (start 160.09874 115.57) (end 159.149999 114.621259) (width 0.8) (layer F.Cu) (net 5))
 (segment (start 163.703 115.57) (end 160.09874 115.57) (width 0.8) (layer F.Cu) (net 5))
 (segment (start 160.09874 115.57) (end 155.01874 120.65) (width 0.8) (layer F.Cu) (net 5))
 (segment (start 163.703 116.586) (end 163.703 115.57) (width 0.35) (layer F.Cu) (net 5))
 (segment (start 157.088378 105.41) (end 159.769342 105.41) (width 0.6) (layer F.Cu) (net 6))
 (segment (start 159.769342 105.41) (end 160.120709 105.058633) (width 0.6) (layer F.Cu) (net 6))
 (segment (start 160.120709 104.468582) (end 160.179342 104.409949) (width 0.6) (layer F.Cu) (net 6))
 (segment (start 160.120709 105.058633) (end 160.120709 104.468582) (width 0.6) (layer F.Cu) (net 6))
 (segment (start 156.04 105.41) (end 157.088378 105.41) (width 0.8) (layer F.Cu) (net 6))
 (segment (start 153.83 104.775) (end 155.405 104.775) (width 0.8) (layer F.Cu) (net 6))
 (segment (start 155.405 104.775) (end 156.04 105.41) (width 0.8) (layer F.Cu) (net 6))
 (segment (start 166.37 101.727) (end 162.823658 101.727) (width 0.8) (layer F.Cu) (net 6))
 (segment (start 162.823658 101.727) (end 160.179342 104.371316) (width 0.8) (layer F.Cu) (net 6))
 (segment (start 160.179342 104.371316) (end 160.179342 104.409949) (width 0.8) (layer F.Cu) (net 6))
 (segment (start 166.37 101.727) (end 166.37 106.045) (width 0.8) (layer F.Cu) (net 6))
 (segment (start 166.37 106.045) (end 168.182999 107.857999) (width 0.8) (layer F.Cu) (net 6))
 (segment (start 168.182999 107.857999) (end 168.501001 107.857999) (width 0.8) (layer F.Cu) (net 6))
 (segment (start 168.91 108.266998) (end 168.91 113.178318) (width 0.8) (layer F.Cu) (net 6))
 (segment (start 168.501001 107.857999) (end 168.91 108.266998) (width 0.8) (layer F.Cu) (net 6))
 (segment (start 168.91 113.178318) (end 169.256001 113.524319) (width 0.8) (layer F.Cu) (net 6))
 (segment (start 169.256001 113.524319) (end 169.256001 115.075681) (width 0.8) (layer F.Cu) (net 6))
 (segment (start 169.256001 115.075681) (end 168.91 115.421682) (width 0.8) (layer F.Cu) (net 6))
 (segment (start 168.91 115.421682) (end 168.91 115.57) (width 0.8) (layer F.Cu) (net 6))
 (segment (start 168.91 115.57) (end 167.64 116.84) (width 0.8) (layer F.Cu) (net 6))
 (segment (start 146.59 100.33) (end 146.44 100.33) (width 0.8) (layer F.Cu) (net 6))
 (segment (start 146.44 100.33) (end 144.109999 97.999999) (width 0.8) (layer F.Cu) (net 6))
 (segment (start 144.109999 97.999999) (end 140.959999 97.999999) (width 0.8) (layer F.Cu) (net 6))
 (segment (start 141.605 118.11) (end 142.24 118.11) (width 0.8) (layer F.Cu) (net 6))
 (segment (start 140.839999 99.785775) (end 139.839991 100.785783) (width 0.8) (layer F.Cu) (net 6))
 (segment (start 140.839999 98.119999) (end 140.839999 99.785775) (width 0.8) (layer F.Cu) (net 6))
 (segment (start 140.959999 97.999999) (end 140.839999 98.119999) (width 0.8) (layer F.Cu) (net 6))
 (segment (start 139.789988 113.114219) (end 140.335 113.659231) (width 0.8) (layer F.Cu) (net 6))
 (segment (start 139.789988 110.528445) (end 139.789988 113.114219) (width 0.8) (layer F.Cu) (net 6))
 (segment (start 139.839991 100.785783) (end 139.839991 100.825009) (width 0.8) (layer F.Cu) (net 6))
 (segment (start 140.335 116.84) (end 141.605 118.11) (width 0.8) (layer F.Cu) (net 6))
 (segment (start 139.7 104.001542) (end 138.789978 104.911564) (width 0.8) (layer F.Cu) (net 6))
 (segment (start 139.7 100.965) (end 139.7 104.001542) (width 0.8) (layer F.Cu) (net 6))
 (segment (start 139.839991 100.825009) (end 139.7 100.965) (width 0.8) (layer F.Cu) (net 6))
 (segment (start 138.789978 104.911564) (end 138.789978 109.528436) (width 0.8) (layer F.Cu) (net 6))
 (segment (start 138.789978 109.528436) (end 139.789988 110.528445) (width 0.8) (layer F.Cu) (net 6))
 (segment (start 140.335 113.659231) (end 140.335 116.84) (width 0.8) (layer F.Cu) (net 6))
 (segment (start 146.59 100.33) (end 146.74 100.33) (width 0.8) (layer F.Cu) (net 6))
 (segment (start 148.190001 98.879999) (end 149 98.879999) (width 0.8) (layer F.Cu) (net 6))
 (segment (start 149 98.879999) (end 149.054999 98.934998) (width 0.8) (layer F.Cu) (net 6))
 (segment (start 146.74 100.33) (end 148.190001 98.879999) (width 0.8) (layer F.Cu) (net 6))
 (segment (start 155.810001 101.694999) (end 153.83 103.675) (width 0.8) (layer F.Cu) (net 6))
 (segment (start 149.054999 98.934998) (end 149.109998 98.879999) (width 0.8) (layer F.Cu) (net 6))
 (segment (start 155.810001 98.999999) (end 155.810001 101.694999) (width 0.8) (layer F.Cu) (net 6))
 (segment (start 149.109998 98.879999) (end 155.690001 98.879999) (width 0.8) (layer F.Cu) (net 6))
 (segment (start 155.690001 98.879999) (end 155.810001 98.999999) (width 0.8) (layer F.Cu) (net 6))
 (segment (start 153.83 103.675) (end 153.83 104.775) (width 0.8) (layer F.Cu) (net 6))
 (segment (start 149.459231 108.585) (end 148.43 108.585) (width 0.8) (layer F.Cu) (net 6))
 (segment (start 151.590011 106.45422) (end 149.459231 108.585) (width 0.8) (layer F.Cu) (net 6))
 (segment (start 151.590011 105.439989) (end 151.590011 106.45422) (width 0.8) (layer F.Cu) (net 6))
 (segment (start 152.255 104.775) (end 151.590011 105.439989) (width 0.8) (layer F.Cu) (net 6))
 (segment (start 153.83 104.775) (end 152.255 104.775) (width 0.8) (layer F.Cu) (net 6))
 (segment (start 142.24 107.22) (end 143.605 108.585) (width 0.8) (layer F.Cu) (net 6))
 (segment (start 143.605 108.585) (end 148.43 108.585) (width 0.8) (layer F.Cu) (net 6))
 (segment (start 166.37 109.093) (end 166.37 113.03) (width 0.8) (layer F.Cu) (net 7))
 (segment (start 166.37 113.03) (end 167.64 114.3) (width 0.8) (layer F.Cu) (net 7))
 (segment (start 161.52114 105.41) (end 162.687 105.41) (width 0.8) (layer F.Cu) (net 7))
 (segment (start 162.687 105.41) (end 166.37 109.093) (width 0.8) (layer F.Cu) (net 7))
 (segment (start 158.21 100.33) (end 158.21 104.15114) (width 0.8) (layer F.Cu) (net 10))
 (segment (start 158.21 104.15114) (end 158.51886 104.46) (width 0.8) (layer F.Cu) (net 10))
 (segment (start 143.89 111.22) (end 142.24 111.22) (width 0.8) (layer F.Cu) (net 8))
 (segment (start 145.193002 111.22) (end 143.89 111.22) (width 0.8) (layer F.Cu) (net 8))
 (segment (start 153.169059 119.196057) (end 145.193002 111.22) (width 0.8) (layer F.Cu) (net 8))
 (segment (start 153.169059 121.537848) (end 153.169059 119.196057) (width 0.8) (layer F.Cu) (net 8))
 (segment (start 154.130892 122.499681) (end 153.169059 121.537848) (width 0.8) (layer F.Cu) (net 8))
 (segment (start 158.170319 122.499681) (end 154.130892 122.499681) (width 0.8) (layer F.Cu) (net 8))
 (segment (start 160.02 120.65) (end 158.170319 122.499681) (width 0.8) (layer F.Cu) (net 8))
 (segment (start 150.59 100.33) (end 154.21 100.33) (width 0.8) (layer F.Cu) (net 9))
 (segment (start 150.59 106.040002) (end 150.59 101.98) (width 0.8) (layer F.Cu) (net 9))
 (segment (start 148.43 107.315) (end 149.315002 107.315) (width 0.8) (layer F.Cu) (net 9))
 (segment (start 149.315002 107.315) (end 150.59 106.040002) (width 0.8) (layer F.Cu) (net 9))
 (segment (start 150.59 101.98) (end 150.59 100.33) (width 0.8) (layer F.Cu) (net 9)))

